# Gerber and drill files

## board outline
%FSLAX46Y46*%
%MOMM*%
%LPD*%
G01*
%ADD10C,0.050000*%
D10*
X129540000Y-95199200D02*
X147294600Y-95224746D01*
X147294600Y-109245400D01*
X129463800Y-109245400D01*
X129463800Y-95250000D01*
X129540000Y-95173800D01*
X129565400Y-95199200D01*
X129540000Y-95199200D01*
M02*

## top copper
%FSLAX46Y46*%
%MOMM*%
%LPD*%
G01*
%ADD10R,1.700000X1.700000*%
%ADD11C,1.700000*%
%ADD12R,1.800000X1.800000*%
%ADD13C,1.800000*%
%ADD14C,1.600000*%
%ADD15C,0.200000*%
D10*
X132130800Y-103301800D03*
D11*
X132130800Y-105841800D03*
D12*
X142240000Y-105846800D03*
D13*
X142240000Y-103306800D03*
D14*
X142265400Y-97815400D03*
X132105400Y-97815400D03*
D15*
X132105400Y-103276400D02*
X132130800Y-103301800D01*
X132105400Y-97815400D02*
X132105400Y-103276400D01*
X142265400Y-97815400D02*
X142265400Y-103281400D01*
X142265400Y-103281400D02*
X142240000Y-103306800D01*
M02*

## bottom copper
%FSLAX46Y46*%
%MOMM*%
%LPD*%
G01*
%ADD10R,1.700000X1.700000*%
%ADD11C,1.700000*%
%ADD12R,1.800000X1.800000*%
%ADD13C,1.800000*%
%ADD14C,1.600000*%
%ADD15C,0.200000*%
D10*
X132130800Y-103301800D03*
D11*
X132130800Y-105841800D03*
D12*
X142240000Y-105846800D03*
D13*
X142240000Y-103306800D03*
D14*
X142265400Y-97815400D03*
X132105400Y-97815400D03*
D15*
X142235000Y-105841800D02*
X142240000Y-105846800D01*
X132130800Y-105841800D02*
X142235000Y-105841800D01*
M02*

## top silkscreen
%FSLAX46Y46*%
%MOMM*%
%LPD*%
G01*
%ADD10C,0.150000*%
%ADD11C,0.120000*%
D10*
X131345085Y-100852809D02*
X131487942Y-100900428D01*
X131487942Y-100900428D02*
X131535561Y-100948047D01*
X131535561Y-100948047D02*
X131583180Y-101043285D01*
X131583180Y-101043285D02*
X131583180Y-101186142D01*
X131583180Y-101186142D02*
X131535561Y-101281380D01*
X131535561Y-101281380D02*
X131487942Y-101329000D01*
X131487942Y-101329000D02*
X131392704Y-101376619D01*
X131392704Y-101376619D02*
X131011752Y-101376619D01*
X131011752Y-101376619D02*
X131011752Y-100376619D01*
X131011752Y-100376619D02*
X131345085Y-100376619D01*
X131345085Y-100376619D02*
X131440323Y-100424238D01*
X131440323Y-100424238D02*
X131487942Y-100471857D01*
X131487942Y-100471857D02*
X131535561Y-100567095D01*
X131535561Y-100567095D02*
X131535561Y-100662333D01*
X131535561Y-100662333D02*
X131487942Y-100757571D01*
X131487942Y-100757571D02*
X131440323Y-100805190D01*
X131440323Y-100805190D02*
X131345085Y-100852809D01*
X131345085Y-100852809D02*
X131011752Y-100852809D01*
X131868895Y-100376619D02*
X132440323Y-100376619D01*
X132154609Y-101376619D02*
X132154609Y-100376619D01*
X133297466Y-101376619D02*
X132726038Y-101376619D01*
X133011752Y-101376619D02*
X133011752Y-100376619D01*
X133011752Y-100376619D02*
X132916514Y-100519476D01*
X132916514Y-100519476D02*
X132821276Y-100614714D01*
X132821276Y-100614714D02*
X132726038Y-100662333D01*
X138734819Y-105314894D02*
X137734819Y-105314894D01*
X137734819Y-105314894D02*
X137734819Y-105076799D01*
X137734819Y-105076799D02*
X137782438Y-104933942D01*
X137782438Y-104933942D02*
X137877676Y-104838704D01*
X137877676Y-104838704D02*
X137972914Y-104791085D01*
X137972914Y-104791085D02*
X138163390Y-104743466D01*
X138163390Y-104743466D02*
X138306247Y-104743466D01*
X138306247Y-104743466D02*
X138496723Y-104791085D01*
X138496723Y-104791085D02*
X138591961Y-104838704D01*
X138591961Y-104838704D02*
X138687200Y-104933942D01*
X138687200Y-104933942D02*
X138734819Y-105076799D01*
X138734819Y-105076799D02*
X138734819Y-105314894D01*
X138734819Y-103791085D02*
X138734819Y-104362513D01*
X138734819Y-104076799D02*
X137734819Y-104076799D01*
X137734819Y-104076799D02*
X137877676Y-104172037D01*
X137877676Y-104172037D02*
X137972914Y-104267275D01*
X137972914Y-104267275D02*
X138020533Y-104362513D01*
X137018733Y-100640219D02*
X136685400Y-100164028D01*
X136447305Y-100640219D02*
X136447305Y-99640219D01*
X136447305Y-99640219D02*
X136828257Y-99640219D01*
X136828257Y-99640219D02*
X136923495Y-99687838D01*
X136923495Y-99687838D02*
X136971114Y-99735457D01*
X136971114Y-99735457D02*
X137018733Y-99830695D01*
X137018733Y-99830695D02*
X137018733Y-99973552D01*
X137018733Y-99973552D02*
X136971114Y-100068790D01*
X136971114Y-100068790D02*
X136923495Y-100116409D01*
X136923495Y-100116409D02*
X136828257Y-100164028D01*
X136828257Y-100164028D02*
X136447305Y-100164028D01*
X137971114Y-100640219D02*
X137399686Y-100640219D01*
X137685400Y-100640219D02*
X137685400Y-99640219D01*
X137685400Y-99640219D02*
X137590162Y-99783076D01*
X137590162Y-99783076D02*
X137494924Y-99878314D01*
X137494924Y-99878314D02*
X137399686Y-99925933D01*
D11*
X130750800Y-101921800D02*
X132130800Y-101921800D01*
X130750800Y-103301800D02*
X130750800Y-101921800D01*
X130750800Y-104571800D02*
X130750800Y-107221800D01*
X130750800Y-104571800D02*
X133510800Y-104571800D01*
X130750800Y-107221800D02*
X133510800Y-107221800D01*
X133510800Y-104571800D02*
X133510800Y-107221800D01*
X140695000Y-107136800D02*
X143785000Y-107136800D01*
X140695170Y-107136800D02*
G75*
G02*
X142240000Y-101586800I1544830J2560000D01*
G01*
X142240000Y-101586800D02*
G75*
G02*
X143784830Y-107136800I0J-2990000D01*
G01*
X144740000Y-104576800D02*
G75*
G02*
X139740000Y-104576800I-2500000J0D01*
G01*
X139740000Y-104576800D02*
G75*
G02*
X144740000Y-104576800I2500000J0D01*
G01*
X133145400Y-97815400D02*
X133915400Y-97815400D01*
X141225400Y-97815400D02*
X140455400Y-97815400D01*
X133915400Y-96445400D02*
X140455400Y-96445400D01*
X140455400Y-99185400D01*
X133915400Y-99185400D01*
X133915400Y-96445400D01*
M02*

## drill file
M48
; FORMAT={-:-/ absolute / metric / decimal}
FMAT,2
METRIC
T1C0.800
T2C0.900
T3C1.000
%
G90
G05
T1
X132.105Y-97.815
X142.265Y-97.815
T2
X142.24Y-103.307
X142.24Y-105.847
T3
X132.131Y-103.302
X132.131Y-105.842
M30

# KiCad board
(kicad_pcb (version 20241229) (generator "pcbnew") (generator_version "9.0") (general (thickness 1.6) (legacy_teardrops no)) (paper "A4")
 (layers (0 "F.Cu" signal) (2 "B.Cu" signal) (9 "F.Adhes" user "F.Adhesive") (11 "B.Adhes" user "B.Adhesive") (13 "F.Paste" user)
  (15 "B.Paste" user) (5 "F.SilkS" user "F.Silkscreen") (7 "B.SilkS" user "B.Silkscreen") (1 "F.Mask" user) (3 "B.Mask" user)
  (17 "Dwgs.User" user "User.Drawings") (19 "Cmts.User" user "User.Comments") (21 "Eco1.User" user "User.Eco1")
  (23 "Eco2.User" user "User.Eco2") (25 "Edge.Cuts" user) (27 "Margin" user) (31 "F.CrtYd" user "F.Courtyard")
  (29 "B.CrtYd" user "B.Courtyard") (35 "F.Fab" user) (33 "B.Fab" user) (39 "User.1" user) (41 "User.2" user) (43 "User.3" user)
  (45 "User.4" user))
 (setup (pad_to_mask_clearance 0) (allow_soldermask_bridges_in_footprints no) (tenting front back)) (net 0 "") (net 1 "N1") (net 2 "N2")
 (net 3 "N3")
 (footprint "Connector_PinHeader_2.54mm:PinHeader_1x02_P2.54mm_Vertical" (layer "F.Cu") (at 132.1308 103.3018)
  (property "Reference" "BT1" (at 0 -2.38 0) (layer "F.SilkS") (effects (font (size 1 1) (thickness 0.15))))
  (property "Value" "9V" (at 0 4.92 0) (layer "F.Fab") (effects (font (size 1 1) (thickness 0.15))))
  (fp_line (start -1.38 -1.38) (end 0 -1.38) (stroke (width 0.12) (type solid)) (layer "F.SilkS"))
  (fp_line (start -1.38 0) (end -1.38 -1.38) (stroke (width 0.12) (type solid)) (layer "F.SilkS"))
  (fp_line (start -1.38 1.27) (end -1.38 3.92) (stroke (width 0.12) (type solid)) (layer "F.SilkS"))
  (fp_line (start -1.38 1.27) (end 1.38 1.27) (stroke (width 0.12) (type solid)) (layer "F.SilkS"))
  (fp_line (start -1.38 3.92) (end 1.38 3.92) (stroke (width 0.12) (type solid)) (layer "F.SilkS"))
  (fp_line (start 1.38 1.27) (end 1.38 3.92) (stroke (width 0.12) (type solid)) (layer "F.SilkS"))
  (pad "1" thru_hole rect (at 0 0) (size 1.7 1.7) (drill 1) (layers "*.Cu" "*.Mask") (remove_unused_layers no) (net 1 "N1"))
  (pad "2" thru_hole circle (at 0 2.54) (size 1.7 1.7) (drill 1) (layers "*.Cu" "*.Mask") (remove_unused_layers no) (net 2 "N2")))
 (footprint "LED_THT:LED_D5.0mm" (layer "F.Cu") (at 142.24 105.8468 90)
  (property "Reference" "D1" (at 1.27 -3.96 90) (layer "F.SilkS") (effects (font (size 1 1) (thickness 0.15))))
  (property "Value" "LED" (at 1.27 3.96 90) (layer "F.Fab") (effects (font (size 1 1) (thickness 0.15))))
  (fp_line (start -1.29 -1.545) (end -1.29 1.545) (stroke (width 0.12) (type solid)) (layer "F.SilkS"))
  (fp_arc (start -1.29 -1.54483) (mid 2.071779 -2.880495) (end 4.26 0) (stroke (width 0.12) (type solid)) (layer "F.SilkS"))
  (fp_arc (start 4.26 0) (mid 2.071779 2.880495) (end -1.29 1.54483) (stroke (width 0.12) (type solid)) (layer "F.SilkS"))
  (fp_circle (center 1.27 0) (end 3.77 0) (stroke (width 0.12) (type solid)) (fill no) (layer "F.SilkS"))
  (pad "1" thru_hole rect (at 0 0 90) (size 1.8 1.8) (drill 0.9) (layers "*.Cu" "*.Mask") (remove_unused_layers no) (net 2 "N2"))
  (pad "2" thru_hole circle (at 2.54 0 90) (size 1.8 1.8) (drill 0.9) (layers "*.Cu" "*.Mask") (remove_unused_layers no) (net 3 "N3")))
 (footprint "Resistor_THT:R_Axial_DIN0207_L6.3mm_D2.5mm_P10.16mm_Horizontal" (layer "F.Cu") (at 142.2654 97.8154 180)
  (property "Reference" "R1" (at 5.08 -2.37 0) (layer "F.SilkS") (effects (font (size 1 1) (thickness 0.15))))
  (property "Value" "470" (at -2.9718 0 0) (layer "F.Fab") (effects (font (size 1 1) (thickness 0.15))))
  (fp_line (start 9.12 0) (end 8.35 0) (stroke (width 0.12) (type solid)) (layer "F.SilkS"))
  (fp_line (start 1.04 0) (end 1.81 0) (stroke (width 0.12) (type solid)) (layer "F.SilkS"))
  (fp_rect (start 1.81 -1.37) (end 8.35 1.37) (stroke (width 0.12) (type solid)) (fill no) (layer "F.SilkS"))
  (pad "1" thru_hole circle (at 0 0 180) (size 1.6 1.6) (drill 0.8) (layers "*.Cu" "*.Mask") (remove_unused_layers no) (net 3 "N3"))
  (pad "2" thru_hole circle (at 10.16 0 180) (size 1.6 1.6) (drill 0.8) (layers "*.Cu" "*.Mask") (remove_unused_layers no) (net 1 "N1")))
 (gr_poly
  (pts (xy 129.54 95.1992) (xy 147.2946 95.224746) (xy 147.2946 109.2454) (xy 129.4638 109.2454) (xy 129.4638 95.25) (xy 129.54 95.1738)
   (xy 129.5654 95.1992))
  (stroke (width 0.05) (type solid)) (fill no) (layer "Edge.Cuts"))
 (segment (start 142.235 105.8418) (end 142.24 105.8468) (width 0.2) (layer "B.Cu") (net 2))
 (segment (start 132.1308 105.8418) (end 142.235 105.8418) (width 0.2) (layer "B.Cu") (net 2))
 (segment (start 132.1054 103.2764) (end 132.1308 103.3018) (width 0.2) (layer "F.Cu") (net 1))
 (segment (start 132.1054 97.8154) (end 132.1054 103.2764) (width 0.2) (layer "F.Cu") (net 1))
 (segment (start 142.2654 97.8154) (end 142.2654 103.2814) (width 0.2) (layer "F.Cu") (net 3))
 (segment (start 142.2654 103.2814) (end 142.24 103.3068) (width 0.2) (layer "F.Cu") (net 3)))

